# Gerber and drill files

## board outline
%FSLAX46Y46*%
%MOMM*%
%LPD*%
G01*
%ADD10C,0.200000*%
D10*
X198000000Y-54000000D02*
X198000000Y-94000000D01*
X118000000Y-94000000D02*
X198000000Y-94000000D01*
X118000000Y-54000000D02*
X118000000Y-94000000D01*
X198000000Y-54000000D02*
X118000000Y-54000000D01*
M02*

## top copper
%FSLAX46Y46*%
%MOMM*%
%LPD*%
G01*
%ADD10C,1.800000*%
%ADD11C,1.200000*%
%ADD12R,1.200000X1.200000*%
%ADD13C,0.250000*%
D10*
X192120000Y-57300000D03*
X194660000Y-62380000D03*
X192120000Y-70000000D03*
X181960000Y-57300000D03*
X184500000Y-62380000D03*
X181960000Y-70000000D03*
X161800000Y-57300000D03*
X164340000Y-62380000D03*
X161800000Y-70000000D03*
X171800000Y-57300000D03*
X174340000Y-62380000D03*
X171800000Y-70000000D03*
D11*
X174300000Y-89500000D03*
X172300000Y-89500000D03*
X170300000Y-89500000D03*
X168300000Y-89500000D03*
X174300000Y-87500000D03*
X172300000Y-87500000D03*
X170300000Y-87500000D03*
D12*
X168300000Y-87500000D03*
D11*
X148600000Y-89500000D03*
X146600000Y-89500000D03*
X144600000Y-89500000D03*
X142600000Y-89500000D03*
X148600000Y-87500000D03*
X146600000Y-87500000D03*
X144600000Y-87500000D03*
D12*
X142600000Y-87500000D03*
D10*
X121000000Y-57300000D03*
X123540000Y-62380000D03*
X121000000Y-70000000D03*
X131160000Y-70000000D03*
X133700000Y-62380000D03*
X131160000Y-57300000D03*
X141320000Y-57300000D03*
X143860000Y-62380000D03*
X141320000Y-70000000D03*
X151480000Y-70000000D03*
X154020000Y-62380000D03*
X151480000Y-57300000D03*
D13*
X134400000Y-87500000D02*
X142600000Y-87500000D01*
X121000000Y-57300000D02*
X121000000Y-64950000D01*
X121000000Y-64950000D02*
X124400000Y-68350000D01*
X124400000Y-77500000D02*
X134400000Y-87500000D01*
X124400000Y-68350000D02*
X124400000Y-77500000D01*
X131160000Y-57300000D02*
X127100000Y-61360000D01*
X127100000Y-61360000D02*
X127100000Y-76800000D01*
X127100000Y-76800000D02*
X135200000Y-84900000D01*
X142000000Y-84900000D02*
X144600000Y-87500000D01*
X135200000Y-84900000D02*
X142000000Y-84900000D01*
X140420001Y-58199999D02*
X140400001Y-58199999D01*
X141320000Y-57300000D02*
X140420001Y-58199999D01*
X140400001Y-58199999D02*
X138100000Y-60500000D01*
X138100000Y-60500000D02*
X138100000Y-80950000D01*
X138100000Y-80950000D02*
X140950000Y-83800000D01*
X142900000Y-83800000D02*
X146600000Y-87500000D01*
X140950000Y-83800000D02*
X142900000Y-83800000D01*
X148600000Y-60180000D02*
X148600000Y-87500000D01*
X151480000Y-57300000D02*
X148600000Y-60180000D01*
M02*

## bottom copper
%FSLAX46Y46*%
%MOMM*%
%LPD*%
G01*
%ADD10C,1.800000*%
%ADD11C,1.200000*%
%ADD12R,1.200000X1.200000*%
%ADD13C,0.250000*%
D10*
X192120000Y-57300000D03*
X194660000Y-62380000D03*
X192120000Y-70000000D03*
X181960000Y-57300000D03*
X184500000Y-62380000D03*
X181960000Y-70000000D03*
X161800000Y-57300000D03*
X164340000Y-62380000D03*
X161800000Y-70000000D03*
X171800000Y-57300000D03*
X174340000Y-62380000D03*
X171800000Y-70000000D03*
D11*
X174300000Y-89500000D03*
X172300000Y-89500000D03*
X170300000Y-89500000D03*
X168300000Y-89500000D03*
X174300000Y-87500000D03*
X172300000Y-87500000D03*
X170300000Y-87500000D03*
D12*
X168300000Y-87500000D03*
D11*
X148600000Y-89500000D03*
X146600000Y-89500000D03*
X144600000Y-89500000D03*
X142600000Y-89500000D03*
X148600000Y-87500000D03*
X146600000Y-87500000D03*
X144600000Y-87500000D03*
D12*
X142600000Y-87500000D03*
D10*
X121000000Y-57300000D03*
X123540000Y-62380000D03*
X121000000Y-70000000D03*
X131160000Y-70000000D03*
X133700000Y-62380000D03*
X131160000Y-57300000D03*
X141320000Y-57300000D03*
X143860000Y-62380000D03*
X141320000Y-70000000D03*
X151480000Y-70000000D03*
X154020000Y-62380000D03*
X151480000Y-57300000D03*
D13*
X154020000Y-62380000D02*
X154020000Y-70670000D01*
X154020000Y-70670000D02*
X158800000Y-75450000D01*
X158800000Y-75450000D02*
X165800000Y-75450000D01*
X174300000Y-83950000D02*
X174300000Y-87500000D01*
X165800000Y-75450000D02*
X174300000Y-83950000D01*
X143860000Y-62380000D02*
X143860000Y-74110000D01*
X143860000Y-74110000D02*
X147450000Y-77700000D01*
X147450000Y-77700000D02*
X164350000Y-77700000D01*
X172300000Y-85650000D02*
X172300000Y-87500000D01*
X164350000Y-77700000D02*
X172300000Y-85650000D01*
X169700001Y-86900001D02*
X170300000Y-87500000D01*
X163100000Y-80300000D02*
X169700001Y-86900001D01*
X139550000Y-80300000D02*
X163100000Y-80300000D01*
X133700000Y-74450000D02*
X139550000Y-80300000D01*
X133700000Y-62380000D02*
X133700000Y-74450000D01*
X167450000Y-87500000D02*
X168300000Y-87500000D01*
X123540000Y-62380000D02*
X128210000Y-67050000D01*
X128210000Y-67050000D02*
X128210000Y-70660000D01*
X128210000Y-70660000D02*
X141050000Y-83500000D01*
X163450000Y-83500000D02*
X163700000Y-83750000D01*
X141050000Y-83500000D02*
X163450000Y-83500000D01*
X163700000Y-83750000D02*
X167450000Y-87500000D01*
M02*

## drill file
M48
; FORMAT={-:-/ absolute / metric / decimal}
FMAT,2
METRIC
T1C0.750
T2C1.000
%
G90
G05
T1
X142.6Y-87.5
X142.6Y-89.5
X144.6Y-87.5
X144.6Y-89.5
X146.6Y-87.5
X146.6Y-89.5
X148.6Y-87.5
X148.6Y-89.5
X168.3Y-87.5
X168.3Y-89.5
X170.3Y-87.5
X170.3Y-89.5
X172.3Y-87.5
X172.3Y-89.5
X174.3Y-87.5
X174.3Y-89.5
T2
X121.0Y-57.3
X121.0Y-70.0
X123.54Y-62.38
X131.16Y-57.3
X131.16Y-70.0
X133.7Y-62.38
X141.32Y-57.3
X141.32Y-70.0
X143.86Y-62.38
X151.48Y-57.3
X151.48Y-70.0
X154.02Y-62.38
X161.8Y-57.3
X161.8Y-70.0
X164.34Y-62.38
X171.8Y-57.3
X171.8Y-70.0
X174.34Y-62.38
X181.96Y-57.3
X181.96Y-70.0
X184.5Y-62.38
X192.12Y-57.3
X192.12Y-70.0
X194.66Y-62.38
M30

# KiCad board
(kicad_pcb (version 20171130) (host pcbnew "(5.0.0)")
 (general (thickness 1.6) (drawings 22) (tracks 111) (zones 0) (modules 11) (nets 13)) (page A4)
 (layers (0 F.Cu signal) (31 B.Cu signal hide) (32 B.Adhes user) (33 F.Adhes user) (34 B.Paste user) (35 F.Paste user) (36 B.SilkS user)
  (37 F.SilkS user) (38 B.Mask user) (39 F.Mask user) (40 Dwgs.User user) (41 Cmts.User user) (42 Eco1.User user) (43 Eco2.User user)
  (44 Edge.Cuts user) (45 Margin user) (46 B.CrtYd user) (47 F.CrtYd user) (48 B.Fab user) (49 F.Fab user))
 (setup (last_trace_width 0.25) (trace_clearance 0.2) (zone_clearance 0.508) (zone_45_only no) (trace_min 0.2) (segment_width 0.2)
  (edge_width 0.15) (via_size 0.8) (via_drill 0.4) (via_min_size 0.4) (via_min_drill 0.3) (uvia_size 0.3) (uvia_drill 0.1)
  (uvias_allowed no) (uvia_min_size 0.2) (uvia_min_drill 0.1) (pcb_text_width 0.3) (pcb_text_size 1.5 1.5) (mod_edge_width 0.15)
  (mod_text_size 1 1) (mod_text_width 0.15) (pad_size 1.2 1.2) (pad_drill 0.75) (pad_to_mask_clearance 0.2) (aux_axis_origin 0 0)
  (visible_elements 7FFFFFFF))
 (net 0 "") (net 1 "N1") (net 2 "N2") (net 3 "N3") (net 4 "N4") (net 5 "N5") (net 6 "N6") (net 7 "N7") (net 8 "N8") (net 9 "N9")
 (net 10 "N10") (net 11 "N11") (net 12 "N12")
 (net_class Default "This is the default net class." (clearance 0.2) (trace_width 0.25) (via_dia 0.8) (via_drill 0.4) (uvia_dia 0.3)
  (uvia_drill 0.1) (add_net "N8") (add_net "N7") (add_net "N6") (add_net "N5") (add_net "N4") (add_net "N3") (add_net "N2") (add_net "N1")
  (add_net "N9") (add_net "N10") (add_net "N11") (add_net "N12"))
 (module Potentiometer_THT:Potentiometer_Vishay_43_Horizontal (layer F.Cu) (at 192.12 70 270)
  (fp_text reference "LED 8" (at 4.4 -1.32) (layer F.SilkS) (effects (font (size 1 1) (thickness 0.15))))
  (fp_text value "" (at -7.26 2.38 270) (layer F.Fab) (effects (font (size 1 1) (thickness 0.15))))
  (pad 3 thru_hole circle (at -12.7 0 270) (size 1.8 1.8) (drill 1) (layers *.Cu *.Mask))
  (pad 2 thru_hole circle (at -7.62 -2.54 270) (size 1.8 1.8) (drill 1) (layers *.Cu *.Mask))
  (pad 1 thru_hole circle (at 0 0 270) (size 1.8 1.8) (drill 1) (layers *.Cu *.Mask)))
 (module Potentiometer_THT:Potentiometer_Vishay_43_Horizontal (layer F.Cu) (at 181.96 70 270)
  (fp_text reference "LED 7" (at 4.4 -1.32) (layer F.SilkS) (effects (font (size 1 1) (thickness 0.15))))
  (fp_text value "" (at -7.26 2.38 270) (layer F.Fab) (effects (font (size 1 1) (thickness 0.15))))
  (pad 3 thru_hole circle (at -12.7 0 270) (size 1.8 1.8) (drill 1) (layers *.Cu *.Mask))
  (pad 2 thru_hole circle (at -7.62 -2.54 270) (size 1.8 1.8) (drill 1) (layers *.Cu *.Mask))
  (pad 1 thru_hole circle (at 0 0 270) (size 1.8 1.8) (drill 1) (layers *.Cu *.Mask)))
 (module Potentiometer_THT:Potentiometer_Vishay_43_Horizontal (layer F.Cu) (at 161.8 70 270)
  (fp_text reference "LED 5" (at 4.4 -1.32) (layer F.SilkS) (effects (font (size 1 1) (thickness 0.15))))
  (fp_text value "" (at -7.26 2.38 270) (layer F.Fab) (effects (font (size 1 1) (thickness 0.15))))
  (pad 3 thru_hole circle (at -12.7 0 270) (size 1.8 1.8) (drill 1) (layers *.Cu *.Mask))
  (pad 2 thru_hole circle (at -7.62 -2.54 270) (size 1.8 1.8) (drill 1) (layers *.Cu *.Mask))
  (pad 1 thru_hole circle (at 0 0 270) (size 1.8 1.8) (drill 1) (layers *.Cu *.Mask)))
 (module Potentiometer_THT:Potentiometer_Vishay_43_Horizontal (layer F.Cu) (at 171.8 70 270)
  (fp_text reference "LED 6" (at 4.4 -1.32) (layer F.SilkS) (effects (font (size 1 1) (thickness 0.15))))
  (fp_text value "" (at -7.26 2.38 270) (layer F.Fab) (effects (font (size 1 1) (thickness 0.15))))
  (pad 3 thru_hole circle (at -12.7 0 270) (size 1.8 1.8) (drill 1) (layers *.Cu *.Mask))
  (pad 2 thru_hole circle (at -7.62 -2.54 270) (size 1.8 1.8) (drill 1) (layers *.Cu *.Mask))
  (pad 1 thru_hole circle (at 0 0 270) (size 1.8 1.8) (drill 1) (layers *.Cu *.Mask)))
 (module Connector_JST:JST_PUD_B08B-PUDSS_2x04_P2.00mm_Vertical (layer F.Cu) (at 168.3 87.5)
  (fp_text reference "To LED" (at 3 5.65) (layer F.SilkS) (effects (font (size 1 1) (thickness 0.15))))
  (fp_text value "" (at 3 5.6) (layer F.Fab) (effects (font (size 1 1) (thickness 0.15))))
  (pad 8 thru_hole circle (at 6 2) (size 1.2 1.2) (drill 0.75) (layers *.Cu *.Mask))
  (pad 6 thru_hole circle (at 4 2) (size 1.2 1.2) (drill 0.75) (layers *.Cu *.Mask))
  (pad 4 thru_hole circle (at 2 2) (size 1.2 1.2) (drill 0.75) (layers *.Cu *.Mask))
  (pad 2 thru_hole circle (at 0 2) (size 1.2 1.2) (drill 0.75) (layers *.Cu *.Mask))
  (pad 7 thru_hole circle (at 6 0) (size 1.2 1.2) (drill 0.75) (layers *.Cu *.Mask) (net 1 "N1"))
  (pad 5 thru_hole circle (at 4 0) (size 1.2 1.2) (drill 0.75) (layers *.Cu *.Mask) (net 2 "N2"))
  (pad 3 thru_hole circle (at 2 0) (size 1.2 1.2) (drill 0.75) (layers *.Cu *.Mask) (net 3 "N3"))
  (pad 1 thru_hole rect (at 0 0) (size 1.2 1.2) (drill 0.75) (layers *.Cu *.Mask) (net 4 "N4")))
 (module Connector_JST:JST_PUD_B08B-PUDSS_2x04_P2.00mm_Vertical (layer F.Cu) (at 142.6 87.5)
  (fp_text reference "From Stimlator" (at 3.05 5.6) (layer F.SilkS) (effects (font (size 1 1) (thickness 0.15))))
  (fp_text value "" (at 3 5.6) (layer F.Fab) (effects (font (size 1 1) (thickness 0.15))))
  (pad 8 thru_hole circle (at 6 2) (size 1.2 1.2) (drill 0.75) (layers *.Cu *.Mask))
  (pad 6 thru_hole circle (at 4 2) (size 1.2 1.2) (drill 0.75) (layers *.Cu *.Mask))
  (pad 4 thru_hole circle (at 2 2) (size 1.2 1.2) (drill 0.75) (layers *.Cu *.Mask))
  (pad 2 thru_hole circle (at 0 2) (size 1.2 1.2) (drill 0.75) (layers *.Cu *.Mask))
  (pad 7 thru_hole circle (at 6 0) (size 1.2 1.2) (drill 0.75) (layers *.Cu *.Mask) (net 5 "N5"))
  (pad 5 thru_hole circle (at 4 0) (size 1.2 1.2) (drill 0.75) (layers *.Cu *.Mask) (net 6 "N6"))
  (pad 3 thru_hole circle (at 2 0) (size 1.2 1.2) (drill 0.75) (layers *.Cu *.Mask) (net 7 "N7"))
  (pad 1 thru_hole rect (at 0 0) (size 1.2 1.2) (drill 0.75) (layers *.Cu *.Mask) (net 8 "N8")))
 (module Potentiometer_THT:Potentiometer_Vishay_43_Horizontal (layer F.Cu) (at 121 70 270)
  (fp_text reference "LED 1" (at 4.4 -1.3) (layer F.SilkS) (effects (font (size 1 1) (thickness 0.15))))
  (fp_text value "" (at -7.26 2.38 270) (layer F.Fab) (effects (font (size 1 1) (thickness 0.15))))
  (pad 3 thru_hole circle (at -12.7 0 270) (size 1.8 1.8) (drill 1) (layers *.Cu *.Mask) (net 8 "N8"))
  (pad 2 thru_hole circle (at -7.62 -2.54 270) (size 1.8 1.8) (drill 1) (layers *.Cu *.Mask) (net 4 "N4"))
  (pad 1 thru_hole circle (at 0 0 270) (size 1.8 1.8) (drill 1) (layers *.Cu *.Mask)))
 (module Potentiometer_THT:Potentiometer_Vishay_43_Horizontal (layer F.Cu) (at 131.16 70 270)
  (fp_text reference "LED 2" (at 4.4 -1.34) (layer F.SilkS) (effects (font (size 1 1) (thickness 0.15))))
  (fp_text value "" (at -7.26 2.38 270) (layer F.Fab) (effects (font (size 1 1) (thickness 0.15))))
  (pad 1 thru_hole circle (at 0 0 270) (size 1.8 1.8) (drill 1) (layers *.Cu *.Mask))
  (pad 2 thru_hole circle (at -7.62 -2.54 270) (size 1.8 1.8) (drill 1) (layers *.Cu *.Mask) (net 3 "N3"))
  (pad 3 thru_hole circle (at -12.7 0 270) (size 1.8 1.8) (drill 1) (layers *.Cu *.Mask) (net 7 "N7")))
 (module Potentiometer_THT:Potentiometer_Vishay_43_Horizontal (layer F.Cu) (at 141.32 70 270)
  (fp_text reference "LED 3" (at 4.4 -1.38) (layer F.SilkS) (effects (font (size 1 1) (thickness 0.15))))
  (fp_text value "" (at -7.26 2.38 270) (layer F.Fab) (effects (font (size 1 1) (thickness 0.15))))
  (pad 3 thru_hole circle (at -12.7 0 270) (size 1.8 1.8) (drill 1) (layers *.Cu *.Mask) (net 6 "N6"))
  (pad 2 thru_hole circle (at -7.62 -2.54 270) (size 1.8 1.8) (drill 1) (layers *.Cu *.Mask) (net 2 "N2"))
  (pad 1 thru_hole circle (at 0 0 270) (size 1.8 1.8) (drill 1) (layers *.Cu *.Mask)))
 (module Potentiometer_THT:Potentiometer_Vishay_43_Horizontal (layer F.Cu) (at 151.48 70 270)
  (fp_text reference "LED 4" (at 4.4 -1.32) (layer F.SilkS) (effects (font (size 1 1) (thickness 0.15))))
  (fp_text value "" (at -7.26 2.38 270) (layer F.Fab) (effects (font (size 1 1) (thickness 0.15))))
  (pad 1 thru_hole circle (at 0 0 270) (size 1.8 1.8) (drill 1) (layers *.Cu *.Mask))
  (pad 2 thru_hole circle (at -7.62 -2.54 270) (size 1.8 1.8) (drill 1) (layers *.Cu *.Mask) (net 1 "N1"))
  (pad 3 thru_hole circle (at -12.7 0 270) (size 1.8 1.8) (drill 1) (layers *.Cu *.Mask) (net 5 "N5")))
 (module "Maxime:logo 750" (layer B.Cu) (at 157.7 76.7 180)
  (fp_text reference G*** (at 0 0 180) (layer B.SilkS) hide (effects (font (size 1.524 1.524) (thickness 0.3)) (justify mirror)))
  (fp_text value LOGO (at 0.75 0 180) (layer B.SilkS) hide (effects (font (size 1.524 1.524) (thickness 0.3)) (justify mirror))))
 (gr_line (start 198 54) (end 198 94) (layer Edge.Cuts) (width 0.2))
 (gr_line (start 118 94) (end 198 94) (layer Edge.Cuts) (width 0.2))
 (gr_line (start 118 54) (end 118 94) (layer Edge.Cuts) (width 0.2))
 (gr_line (start 198 54) (end 118 54) (layer Edge.Cuts) (width 0.2))
 (segment (start 134.4 87.5) (end 142.6 87.5) (width 0.25) (layer F.Cu) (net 8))
 (segment (start 121 57.3) (end 121 64.95) (width 0.25) (layer F.Cu) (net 8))
 (segment (start 121 64.95) (end 124.4 68.35) (width 0.25) (layer F.Cu) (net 8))
 (segment (start 124.4 77.5) (end 134.4 87.5) (width 0.25) (layer F.Cu) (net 8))
 (segment (start 124.4 68.35) (end 124.4 77.5) (width 0.25) (layer F.Cu) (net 8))
 (segment (start 131.16 57.3) (end 127.1 61.36) (width 0.25) (layer F.Cu) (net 7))
 (segment (start 127.1 61.36) (end 127.1 76.8) (width 0.25) (layer F.Cu) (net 7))
 (segment (start 127.1 76.8) (end 135.2 84.9) (width 0.25) (layer F.Cu) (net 7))
 (segment (start 142 84.9) (end 144.6 87.5) (width 0.25) (layer F.Cu) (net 7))
 (segment (start 135.2 84.9) (end 142 84.9) (width 0.25) (layer F.Cu) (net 7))
 (segment (start 140.420001 58.199999) (end 140.400001 58.199999) (width 0.25) (layer F.Cu) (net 6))
 (segment (start 141.32 57.3) (end 140.420001 58.199999) (width 0.25) (layer F.Cu) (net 6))
 (segment (start 140.400001 58.199999) (end 138.1 60.5) (width 0.25) (layer F.Cu) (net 6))
 (segment (start 138.1 60.5) (end 138.1 80.95) (width 0.25) (layer F.Cu) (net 6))
 (segment (start 138.1 80.95) (end 140.95 83.8) (width 0.25) (layer F.Cu) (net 6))
 (segment (start 142.9 83.8) (end 146.6 87.5) (width 0.25) (layer F.Cu) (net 6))
 (segment (start 140.95 83.8) (end 142.9 83.8) (width 0.25) (layer F.Cu) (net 6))
 (segment (start 148.6 60.18) (end 148.6 87.5) (width 0.25) (layer F.Cu) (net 5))
 (segment (start 151.48 57.3) (end 148.6 60.18) (width 0.25) (layer F.Cu) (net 5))
 (segment (start 154.02 62.38) (end 154.02 70.67) (width 0.25) (layer B.Cu) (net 1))
 (segment (start 154.02 70.67) (end 158.8 75.45) (width 0.25) (layer B.Cu) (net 1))
 (segment (start 158.8 75.45) (end 165.8 75.45) (width 0.25) (layer B.Cu) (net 1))
 (segment (start 174.3 83.95) (end 174.3 87.5) (width 0.25) (layer B.Cu) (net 1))
 (segment (start 165.8 75.45) (end 174.3 83.95) (width 0.25) (layer B.Cu) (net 1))
 (segment (start 143.86 62.38) (end 143.86 74.11) (width 0.25) (layer B.Cu) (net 2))
 (segment (start 143.86 74.11) (end 147.45 77.7) (width 0.25) (layer B.Cu) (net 2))
 (segment (start 147.45 77.7) (end 164.35 77.7) (width 0.25) (layer B.Cu) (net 2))
 (segment (start 172.3 85.65) (end 172.3 87.5) (width 0.25) (layer B.Cu) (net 2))
 (segment (start 164.35 77.7) (end 172.3 85.65) (width 0.25) (layer B.Cu) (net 2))
 (segment (start 169.700001 86.900001) (end 170.3 87.5) (width 0.25) (layer B.Cu) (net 3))
 (segment (start 163.1 80.3) (end 169.700001 86.900001) (width 0.25) (layer B.Cu) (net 3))
 (segment (start 139.55 80.3) (end 163.1 80.3) (width 0.25) (layer B.Cu) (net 3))
 (segment (start 133.7 74.45) (end 139.55 80.3) (width 0.25) (layer B.Cu) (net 3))
 (segment (start 133.7 62.38) (end 133.7 74.45) (width 0.25) (layer B.Cu) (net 3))
 (segment (start 167.45 87.5) (end 168.3 87.5) (width 0.25) (layer B.Cu) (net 4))
 (segment (start 123.54 62.38) (end 128.21 67.05) (width 0.25) (layer B.Cu) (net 4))
 (segment (start 128.21 67.05) (end 128.21 70.66) (width 0.25) (layer B.Cu) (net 4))
 (segment (start 128.21 70.66) (end 141.05 83.5) (width 0.25) (layer B.Cu) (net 4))
 (segment (start 163.45 83.5) (end 163.7 83.75) (width 0.25) (layer B.Cu) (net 4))
 (segment (start 141.05 83.5) (end 163.45 83.5) (width 0.25) (layer B.Cu) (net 4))
 (segment (start 163.7 83.75) (end 167.45 87.5) (width 0.25) (layer B.Cu) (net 4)))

